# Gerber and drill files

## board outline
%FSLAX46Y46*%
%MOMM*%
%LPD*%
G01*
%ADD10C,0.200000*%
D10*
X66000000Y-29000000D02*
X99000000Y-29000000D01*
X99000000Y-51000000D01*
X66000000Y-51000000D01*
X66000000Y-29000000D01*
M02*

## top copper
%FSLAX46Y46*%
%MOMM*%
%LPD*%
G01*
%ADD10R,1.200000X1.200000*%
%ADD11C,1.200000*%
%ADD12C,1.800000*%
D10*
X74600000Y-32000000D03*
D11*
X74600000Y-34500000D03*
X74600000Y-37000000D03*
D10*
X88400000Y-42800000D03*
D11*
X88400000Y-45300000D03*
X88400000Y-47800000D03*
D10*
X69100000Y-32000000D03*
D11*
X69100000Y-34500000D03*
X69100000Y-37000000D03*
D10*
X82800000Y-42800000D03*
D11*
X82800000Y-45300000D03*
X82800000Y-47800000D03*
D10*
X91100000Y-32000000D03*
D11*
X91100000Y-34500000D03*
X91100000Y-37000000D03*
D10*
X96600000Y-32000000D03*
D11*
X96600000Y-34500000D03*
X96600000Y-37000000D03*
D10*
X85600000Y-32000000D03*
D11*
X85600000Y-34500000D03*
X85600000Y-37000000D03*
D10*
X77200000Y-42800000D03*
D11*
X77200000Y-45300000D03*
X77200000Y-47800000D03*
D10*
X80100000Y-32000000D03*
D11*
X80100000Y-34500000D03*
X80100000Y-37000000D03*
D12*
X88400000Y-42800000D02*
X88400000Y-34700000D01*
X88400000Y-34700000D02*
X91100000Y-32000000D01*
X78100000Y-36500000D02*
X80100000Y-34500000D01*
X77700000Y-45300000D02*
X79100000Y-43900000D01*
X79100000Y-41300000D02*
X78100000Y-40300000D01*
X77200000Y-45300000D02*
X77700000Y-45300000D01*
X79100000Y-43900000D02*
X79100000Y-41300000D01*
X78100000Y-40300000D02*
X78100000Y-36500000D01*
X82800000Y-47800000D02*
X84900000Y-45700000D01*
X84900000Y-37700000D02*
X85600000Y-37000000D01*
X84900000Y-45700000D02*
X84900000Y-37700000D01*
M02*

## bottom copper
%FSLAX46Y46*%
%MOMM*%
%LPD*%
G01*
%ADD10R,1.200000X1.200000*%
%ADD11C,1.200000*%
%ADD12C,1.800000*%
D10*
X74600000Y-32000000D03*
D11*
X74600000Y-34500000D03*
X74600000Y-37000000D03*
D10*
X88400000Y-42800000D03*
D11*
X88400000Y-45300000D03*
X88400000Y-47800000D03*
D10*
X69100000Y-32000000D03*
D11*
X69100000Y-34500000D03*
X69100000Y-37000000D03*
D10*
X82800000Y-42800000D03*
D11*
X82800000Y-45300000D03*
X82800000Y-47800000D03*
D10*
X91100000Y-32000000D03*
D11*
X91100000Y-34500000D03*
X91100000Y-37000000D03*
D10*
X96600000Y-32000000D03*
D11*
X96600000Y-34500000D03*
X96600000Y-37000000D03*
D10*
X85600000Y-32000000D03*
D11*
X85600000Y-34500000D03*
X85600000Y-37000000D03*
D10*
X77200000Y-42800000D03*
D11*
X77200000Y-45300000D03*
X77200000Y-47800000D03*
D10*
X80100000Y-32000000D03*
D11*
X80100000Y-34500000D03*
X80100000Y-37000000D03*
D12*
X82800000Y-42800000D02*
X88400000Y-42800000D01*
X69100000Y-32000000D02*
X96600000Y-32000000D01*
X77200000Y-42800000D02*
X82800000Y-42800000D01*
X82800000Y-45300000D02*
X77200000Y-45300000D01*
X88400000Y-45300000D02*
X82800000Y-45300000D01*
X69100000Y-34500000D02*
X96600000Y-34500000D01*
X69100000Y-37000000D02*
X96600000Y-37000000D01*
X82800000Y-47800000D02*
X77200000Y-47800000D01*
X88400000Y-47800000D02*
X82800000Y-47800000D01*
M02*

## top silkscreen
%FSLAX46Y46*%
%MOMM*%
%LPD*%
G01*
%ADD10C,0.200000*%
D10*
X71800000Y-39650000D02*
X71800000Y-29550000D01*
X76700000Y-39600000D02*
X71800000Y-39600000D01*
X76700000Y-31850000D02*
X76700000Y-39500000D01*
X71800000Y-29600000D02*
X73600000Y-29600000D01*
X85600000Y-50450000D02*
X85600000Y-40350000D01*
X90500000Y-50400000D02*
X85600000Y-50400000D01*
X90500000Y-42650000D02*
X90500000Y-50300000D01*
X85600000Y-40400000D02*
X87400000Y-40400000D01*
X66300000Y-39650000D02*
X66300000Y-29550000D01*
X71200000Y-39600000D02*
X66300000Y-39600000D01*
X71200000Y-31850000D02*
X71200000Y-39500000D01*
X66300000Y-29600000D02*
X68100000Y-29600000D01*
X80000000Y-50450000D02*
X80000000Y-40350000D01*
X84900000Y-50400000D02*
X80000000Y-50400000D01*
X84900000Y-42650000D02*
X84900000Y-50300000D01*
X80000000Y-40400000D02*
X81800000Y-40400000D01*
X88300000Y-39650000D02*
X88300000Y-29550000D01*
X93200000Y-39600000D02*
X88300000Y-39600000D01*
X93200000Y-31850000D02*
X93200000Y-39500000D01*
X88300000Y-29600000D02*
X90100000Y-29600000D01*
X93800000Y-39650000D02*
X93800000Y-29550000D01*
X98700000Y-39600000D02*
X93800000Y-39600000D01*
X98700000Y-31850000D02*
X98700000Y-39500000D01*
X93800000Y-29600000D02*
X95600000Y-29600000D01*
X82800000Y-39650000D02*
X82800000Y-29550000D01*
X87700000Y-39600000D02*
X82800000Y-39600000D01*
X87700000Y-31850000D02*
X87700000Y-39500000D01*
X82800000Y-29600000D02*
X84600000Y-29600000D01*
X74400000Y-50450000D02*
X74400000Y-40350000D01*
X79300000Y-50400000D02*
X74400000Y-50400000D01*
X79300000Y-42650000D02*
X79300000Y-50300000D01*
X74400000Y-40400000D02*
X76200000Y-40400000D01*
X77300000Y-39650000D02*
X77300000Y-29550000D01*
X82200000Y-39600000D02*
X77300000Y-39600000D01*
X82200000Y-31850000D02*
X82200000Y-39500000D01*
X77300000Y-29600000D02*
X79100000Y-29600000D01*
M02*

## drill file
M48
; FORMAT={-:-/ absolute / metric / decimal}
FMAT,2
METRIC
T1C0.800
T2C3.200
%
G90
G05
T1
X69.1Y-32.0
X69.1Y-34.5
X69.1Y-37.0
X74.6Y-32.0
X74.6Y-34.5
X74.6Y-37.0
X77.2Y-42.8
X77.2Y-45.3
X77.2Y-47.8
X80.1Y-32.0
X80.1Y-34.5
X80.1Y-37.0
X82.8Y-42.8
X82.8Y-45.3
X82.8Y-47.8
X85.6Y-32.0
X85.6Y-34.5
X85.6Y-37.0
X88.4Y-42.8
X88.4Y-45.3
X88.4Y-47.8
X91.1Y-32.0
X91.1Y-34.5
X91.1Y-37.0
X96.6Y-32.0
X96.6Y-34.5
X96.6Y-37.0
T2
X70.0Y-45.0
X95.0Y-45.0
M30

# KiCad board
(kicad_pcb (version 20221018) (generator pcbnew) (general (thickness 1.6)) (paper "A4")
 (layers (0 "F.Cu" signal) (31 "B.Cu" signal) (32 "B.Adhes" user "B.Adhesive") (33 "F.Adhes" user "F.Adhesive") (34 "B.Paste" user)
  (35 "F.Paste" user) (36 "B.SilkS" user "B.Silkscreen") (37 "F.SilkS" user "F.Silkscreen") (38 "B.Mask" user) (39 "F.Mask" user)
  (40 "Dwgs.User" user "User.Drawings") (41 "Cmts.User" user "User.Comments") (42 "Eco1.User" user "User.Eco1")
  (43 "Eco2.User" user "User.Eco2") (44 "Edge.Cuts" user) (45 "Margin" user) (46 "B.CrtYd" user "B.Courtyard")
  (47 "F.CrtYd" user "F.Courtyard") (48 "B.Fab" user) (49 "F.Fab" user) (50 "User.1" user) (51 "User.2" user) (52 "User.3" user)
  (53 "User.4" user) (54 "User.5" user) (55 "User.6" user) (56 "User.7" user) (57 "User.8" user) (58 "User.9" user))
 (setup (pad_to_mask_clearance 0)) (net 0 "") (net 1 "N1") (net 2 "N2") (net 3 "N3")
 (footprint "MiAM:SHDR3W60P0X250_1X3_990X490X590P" (layer "F.Cu") (at 74.6 32 90)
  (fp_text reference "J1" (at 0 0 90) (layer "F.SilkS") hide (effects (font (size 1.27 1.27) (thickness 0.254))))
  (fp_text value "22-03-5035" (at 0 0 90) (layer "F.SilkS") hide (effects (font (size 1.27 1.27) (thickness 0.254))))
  (fp_line (start -7.65 -2.8) (end 2.45 -2.8) (stroke (width 0.2) (type solid)) (layer "F.SilkS"))
  (fp_line (start -7.6 2.1) (end -7.6 -2.8) (stroke (width 0.2) (type solid)) (layer "F.SilkS"))
  (fp_line (start 0.15 2.1) (end -7.5 2.1) (stroke (width 0.2) (type solid)) (layer "F.SilkS"))
  (fp_line (start 2.4 -2.8) (end 2.4 -1) (stroke (width 0.2) (type solid)) (layer "F.SilkS"))
  (pad "1" thru_hole rect (at 0 0 90) (size 1.2 1.2) (drill 0.8) (layers "*.Cu" "*.Mask") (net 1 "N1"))
  (pad "2" thru_hole circle (at -2.5 0 90) (size 1.2 1.2) (drill 0.8) (layers "*.Cu" "*.Mask") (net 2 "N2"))
  (pad "3" thru_hole circle (at -5 0 90) (size 1.2 1.2) (drill 0.8) (layers "*.Cu" "*.Mask") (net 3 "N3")))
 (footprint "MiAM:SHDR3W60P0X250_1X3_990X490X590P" (layer "F.Cu") (at 88.4 42.8 90)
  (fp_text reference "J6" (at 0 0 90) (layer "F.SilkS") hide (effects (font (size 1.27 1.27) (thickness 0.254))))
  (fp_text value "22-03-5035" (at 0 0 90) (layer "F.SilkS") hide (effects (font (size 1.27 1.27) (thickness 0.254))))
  (fp_line (start -7.65 -2.8) (end 2.45 -2.8) (stroke (width 0.2) (type solid)) (layer "F.SilkS"))
  (fp_line (start -7.6 2.1) (end -7.6 -2.8) (stroke (width 0.2) (type solid)) (layer "F.SilkS"))
  (fp_line (start 0.15 2.1) (end -7.5 2.1) (stroke (width 0.2) (type solid)) (layer "F.SilkS"))
  (fp_line (start 2.4 -2.8) (end 2.4 -1) (stroke (width 0.2) (type solid)) (layer "F.SilkS"))
  (pad "1" thru_hole rect (at 0 0 90) (size 1.2 1.2) (drill 0.8) (layers "*.Cu" "*.Mask") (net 1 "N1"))
  (pad "2" thru_hole circle locked (at -2.5 0 90) (size 1.2 1.2) (drill 0.8) (layers "*.Cu" "*.Mask") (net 2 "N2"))
  (pad "3" thru_hole circle (at -5 0 90) (size 1.2 1.2) (drill 0.8) (layers "*.Cu" "*.Mask") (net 3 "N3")))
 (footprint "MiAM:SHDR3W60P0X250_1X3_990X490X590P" (layer "F.Cu") (at 69.1 32 90)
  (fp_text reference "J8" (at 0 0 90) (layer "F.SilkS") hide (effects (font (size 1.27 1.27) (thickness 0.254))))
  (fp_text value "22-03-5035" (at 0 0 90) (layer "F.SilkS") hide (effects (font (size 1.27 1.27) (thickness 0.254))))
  (fp_line (start -7.65 -2.8) (end 2.45 -2.8) (stroke (width 0.2) (type solid)) (layer "F.SilkS"))
  (fp_line (start -7.6 2.1) (end -7.6 -2.8) (stroke (width 0.2) (type solid)) (layer "F.SilkS"))
  (fp_line (start 0.15 2.1) (end -7.5 2.1) (stroke (width 0.2) (type solid)) (layer "F.SilkS"))
  (fp_line (start 2.4 -2.8) (end 2.4 -1) (stroke (width 0.2) (type solid)) (layer "F.SilkS"))
  (pad "1" thru_hole rect (at 0 0 90) (size 1.2 1.2) (drill 0.8) (layers "*.Cu" "*.Mask") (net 1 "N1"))
  (pad "2" thru_hole circle (at -2.5 0 90) (size 1.2 1.2) (drill 0.8) (layers "*.Cu" "*.Mask") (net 2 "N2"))
  (pad "3" thru_hole circle (at -5 0 90) (size 1.2 1.2) (drill 0.8) (layers "*.Cu" "*.Mask") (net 3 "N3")))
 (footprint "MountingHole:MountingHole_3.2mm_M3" (layer "F.Cu") (at 70 45)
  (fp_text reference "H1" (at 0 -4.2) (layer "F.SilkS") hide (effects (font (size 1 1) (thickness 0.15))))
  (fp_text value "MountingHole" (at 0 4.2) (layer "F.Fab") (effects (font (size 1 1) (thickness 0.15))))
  (pad "" np_thru_hole circle (at 0 0) (size 3.2 3.2) (drill 3.2) (layers "*.Cu" "*.Mask")))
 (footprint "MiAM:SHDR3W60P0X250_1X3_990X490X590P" (layer "F.Cu") (at 82.8 42.8 90)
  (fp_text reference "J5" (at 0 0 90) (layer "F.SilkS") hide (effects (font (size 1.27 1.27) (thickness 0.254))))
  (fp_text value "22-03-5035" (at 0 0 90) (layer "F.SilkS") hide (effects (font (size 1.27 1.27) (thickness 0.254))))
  (fp_line (start -7.65 -2.8) (end 2.45 -2.8) (stroke (width 0.2) (type solid)) (layer "F.SilkS"))
  (fp_line (start -7.6 2.1) (end -7.6 -2.8) (stroke (width 0.2) (type solid)) (layer "F.SilkS"))
  (fp_line (start 0.15 2.1) (end -7.5 2.1) (stroke (width 0.2) (type solid)) (layer "F.SilkS"))
  (fp_line (start 2.4 -2.8) (end 2.4 -1) (stroke (width 0.2) (type solid)) (layer "F.SilkS"))
  (pad "1" thru_hole rect (at 0 0 90) (size 1.2 1.2) (drill 0.8) (layers "*.Cu" "*.Mask") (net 1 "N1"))
  (pad "2" thru_hole circle (at -2.5 0 90) (size 1.2 1.2) (drill 0.8) (layers "*.Cu" "*.Mask") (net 2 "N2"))
  (pad "3" thru_hole circle (at -5 0 90) (size 1.2 1.2) (drill 0.8) (layers "*.Cu" "*.Mask") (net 3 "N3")))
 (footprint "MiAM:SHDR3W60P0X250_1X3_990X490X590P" (layer "F.Cu") (at 91.1 32 90)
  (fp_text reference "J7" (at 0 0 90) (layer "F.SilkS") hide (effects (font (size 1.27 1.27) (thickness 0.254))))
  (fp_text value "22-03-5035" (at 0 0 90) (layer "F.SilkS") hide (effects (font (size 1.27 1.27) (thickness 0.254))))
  (fp_line (start -7.65 -2.8) (end 2.45 -2.8) (stroke (width 0.2) (type solid)) (layer "F.SilkS"))
  (fp_line (start -7.6 2.1) (end -7.6 -2.8) (stroke (width 0.2) (type solid)) (layer "F.SilkS"))
  (fp_line (start 0.15 2.1) (end -7.5 2.1) (stroke (width 0.2) (type solid)) (layer "F.SilkS"))
  (fp_line (start 2.4 -2.8) (end 2.4 -1) (stroke (width 0.2) (type solid)) (layer "F.SilkS"))
  (pad "1" thru_hole rect (at 0 0 90) (size 1.2 1.2) (drill 0.8) (layers "*.Cu" "*.Mask") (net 1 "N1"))
  (pad "2" thru_hole circle (at -2.5 0 90) (size 1.2 1.2) (drill 0.8) (layers "*.Cu" "*.Mask") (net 2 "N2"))
  (pad "3" thru_hole circle (at -5 0 90) (size 1.2 1.2) (drill 0.8) (layers "*.Cu" "*.Mask") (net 3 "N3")))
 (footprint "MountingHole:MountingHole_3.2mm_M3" (layer "F.Cu") (at 95 45)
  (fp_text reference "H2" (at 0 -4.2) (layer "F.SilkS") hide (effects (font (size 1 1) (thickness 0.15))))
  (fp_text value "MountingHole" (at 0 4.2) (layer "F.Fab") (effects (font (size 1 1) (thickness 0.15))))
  (pad "" np_thru_hole circle (at 0 0) (size 3.2 3.2) (drill 3.2) (layers "*.Cu" "*.Mask")))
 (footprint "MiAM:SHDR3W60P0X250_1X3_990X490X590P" (layer "F.Cu") (at 96.6 32 90)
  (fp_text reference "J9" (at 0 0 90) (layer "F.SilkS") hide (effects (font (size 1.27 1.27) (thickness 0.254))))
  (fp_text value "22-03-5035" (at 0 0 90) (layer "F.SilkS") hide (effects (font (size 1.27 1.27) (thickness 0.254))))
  (fp_line (start -7.65 -2.8) (end 2.45 -2.8) (stroke (width 0.2) (type solid)) (layer "F.SilkS"))
  (fp_line (start -7.6 2.1) (end -7.6 -2.8) (stroke (width 0.2) (type solid)) (layer "F.SilkS"))
  (fp_line (start 0.15 2.1) (end -7.5 2.1) (stroke (width 0.2) (type solid)) (layer "F.SilkS"))
  (fp_line (start 2.4 -2.8) (end 2.4 -1) (stroke (width 0.2) (type solid)) (layer "F.SilkS"))
  (pad "1" thru_hole rect (at 0 0 90) (size 1.2 1.2) (drill 0.8) (layers "*.Cu" "*.Mask") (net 1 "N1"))
  (pad "2" thru_hole circle (at -2.5 0 90) (size 1.2 1.2) (drill 0.8) (layers "*.Cu" "*.Mask") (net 2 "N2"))
  (pad "3" thru_hole circle (at -5 0 90) (size 1.2 1.2) (drill 0.8) (layers "*.Cu" "*.Mask") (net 3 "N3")))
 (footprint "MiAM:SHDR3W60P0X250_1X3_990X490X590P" (layer "F.Cu") (at 85.6 32 90)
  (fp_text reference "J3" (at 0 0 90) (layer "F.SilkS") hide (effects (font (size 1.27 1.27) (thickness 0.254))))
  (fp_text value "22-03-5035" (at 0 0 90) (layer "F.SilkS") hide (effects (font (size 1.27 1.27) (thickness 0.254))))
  (fp_line (start -7.65 -2.8) (end 2.45 -2.8) (stroke (width 0.2) (type solid)) (layer "F.SilkS"))
  (fp_line (start -7.6 2.1) (end -7.6 -2.8) (stroke (width 0.2) (type solid)) (layer "F.SilkS"))
  (fp_line (start 0.15 2.1) (end -7.5 2.1) (stroke (width 0.2) (type solid)) (layer "F.SilkS"))
  (fp_line (start 2.4 -2.8) (end 2.4 -1) (stroke (width 0.2) (type solid)) (layer "F.SilkS"))
  (pad "1" thru_hole rect (at 0 0 90) (size 1.2 1.2) (drill 0.8) (layers "*.Cu" "*.Mask") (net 1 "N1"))
  (pad "2" thru_hole circle (at -2.5 0 90) (size 1.2 1.2) (drill 0.8) (layers "*.Cu" "*.Mask") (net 2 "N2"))
  (pad "3" thru_hole circle (at -5 0 90) (size 1.2 1.2) (drill 0.8) (layers "*.Cu" "*.Mask") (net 3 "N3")))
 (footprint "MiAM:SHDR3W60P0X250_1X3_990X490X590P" (layer "F.Cu") (at 77.2 42.8 90)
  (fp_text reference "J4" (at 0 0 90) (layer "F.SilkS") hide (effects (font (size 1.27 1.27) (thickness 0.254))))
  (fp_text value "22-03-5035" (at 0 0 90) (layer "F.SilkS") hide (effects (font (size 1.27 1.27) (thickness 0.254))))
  (fp_line (start -7.65 -2.8) (end 2.45 -2.8) (stroke (width 0.2) (type solid)) (layer "F.SilkS"))
  (fp_line (start -7.6 2.1) (end -7.6 -2.8) (stroke (width 0.2) (type solid)) (layer "F.SilkS"))
  (fp_line (start 0.15 2.1) (end -7.5 2.1) (stroke (width 0.2) (type solid)) (layer "F.SilkS"))
  (fp_line (start 2.4 -2.8) (end 2.4 -1) (stroke (width 0.2) (type solid)) (layer "F.SilkS"))
  (pad "1" thru_hole rect (at 0 0 90) (size 1.2 1.2) (drill 0.8) (layers "*.Cu" "*.Mask") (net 1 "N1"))
  (pad "2" thru_hole circle (at -2.5 0 90) (size 1.2 1.2) (drill 0.8) (layers "*.Cu" "*.Mask") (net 2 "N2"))
  (pad "3" thru_hole circle (at -5 0 90) (size 1.2 1.2) (drill 0.8) (layers "*.Cu" "*.Mask") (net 3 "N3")))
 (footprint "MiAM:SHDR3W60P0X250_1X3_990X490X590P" (layer "F.Cu") (at 80.1 32 90)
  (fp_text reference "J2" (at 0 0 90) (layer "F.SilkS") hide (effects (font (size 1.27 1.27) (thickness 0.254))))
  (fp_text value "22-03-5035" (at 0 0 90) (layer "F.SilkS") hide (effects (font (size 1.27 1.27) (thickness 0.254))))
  (fp_line (start -7.65 -2.8) (end 2.45 -2.8) (stroke (width 0.2) (type solid)) (layer "F.SilkS"))
  (fp_line (start -7.6 2.1) (end -7.6 -2.8) (stroke (width 0.2) (type solid)) (layer "F.SilkS"))
  (fp_line (start 0.15 2.1) (end -7.5 2.1) (stroke (width 0.2) (type solid)) (layer "F.SilkS"))
  (fp_line (start 2.4 -2.8) (end 2.4 -1) (stroke (width 0.2) (type solid)) (layer "F.SilkS"))
  (pad "1" thru_hole rect (at 0 0 90) (size 1.2 1.2) (drill 0.8) (layers "*.Cu" "*.Mask") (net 1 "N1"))
  (pad "2" thru_hole circle (at -2.5 0 90) (size 1.2 1.2) (drill 0.8) (layers "*.Cu" "*.Mask") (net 2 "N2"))
  (pad "3" thru_hole circle (at -5 0 90) (size 1.2 1.2) (drill 0.8) (layers "*.Cu" "*.Mask") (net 3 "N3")))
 (gr_rect (start 66 29) (end 99 51) (stroke (width 0.2) (type default)) (fill none) (layer "Edge.Cuts"))
 (segment (start 88.4 42.8) (end 88.4 34.7) (width 1.8) (layer "F.Cu") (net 1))
 (segment (start 88.4 34.7) (end 91.1 32) (width 1.8) (layer "F.Cu") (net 1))
 (segment (start 82.8 42.8) (end 88.4 42.8) (width 1.8) (layer "B.Cu") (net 1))
 (segment (start 69.1 32) (end 96.6 32) (width 1.8) (layer "B.Cu") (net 1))
 (segment (start 77.2 42.8) (end 82.8 42.8) (width 1.8) (layer "B.Cu") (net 1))
 (segment (start 78.1 36.5) (end 80.1 34.5) (width 1.8) (layer "F.Cu") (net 2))
 (segment (start 77.7 45.3) (end 79.1 43.9) (width 1.8) (layer "F.Cu") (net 2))
 (segment (start 79.1 41.3) (end 78.1 40.3) (width 1.8) (layer "F.Cu") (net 2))
 (segment (start 77.2 45.3) (end 77.7 45.3) (width 1.8) (layer "F.Cu") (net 2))
 (segment (start 79.1 43.9) (end 79.1 41.3) (width 1.8) (layer "F.Cu") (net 2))
 (segment (start 78.1 40.3) (end 78.1 36.5) (width 1.8) (layer "F.Cu") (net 2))
 (segment (start 82.8 45.3) (end 77.2 45.3) (width 1.8) (layer "B.Cu") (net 2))
 (segment (start 88.4 45.3) (end 82.8 45.3) (width 1.8) (layer "B.Cu") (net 2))
 (segment (start 69.1 34.5) (end 96.6 34.5) (width 1.8) (layer "B.Cu") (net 2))
 (segment (start 82.8 47.8) (end 84.9 45.7) (width 1.8) (layer "F.Cu") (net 3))
 (segment (start 84.9 37.7) (end 85.6 37) (width 1.8) (layer "F.Cu") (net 3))
 (segment (start 84.9 45.7) (end 84.9 37.7) (width 1.8) (layer "F.Cu") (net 3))
 (segment (start 69.1 37) (end 96.6 37) (width 1.8) (layer "B.Cu") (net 3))
 (segment (start 82.8 47.8) (end 77.2 47.8) (width 1.8) (layer "B.Cu") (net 3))
 (segment (start 88.4 47.8) (end 82.8 47.8) (width 1.8) (layer "B.Cu") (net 3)))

